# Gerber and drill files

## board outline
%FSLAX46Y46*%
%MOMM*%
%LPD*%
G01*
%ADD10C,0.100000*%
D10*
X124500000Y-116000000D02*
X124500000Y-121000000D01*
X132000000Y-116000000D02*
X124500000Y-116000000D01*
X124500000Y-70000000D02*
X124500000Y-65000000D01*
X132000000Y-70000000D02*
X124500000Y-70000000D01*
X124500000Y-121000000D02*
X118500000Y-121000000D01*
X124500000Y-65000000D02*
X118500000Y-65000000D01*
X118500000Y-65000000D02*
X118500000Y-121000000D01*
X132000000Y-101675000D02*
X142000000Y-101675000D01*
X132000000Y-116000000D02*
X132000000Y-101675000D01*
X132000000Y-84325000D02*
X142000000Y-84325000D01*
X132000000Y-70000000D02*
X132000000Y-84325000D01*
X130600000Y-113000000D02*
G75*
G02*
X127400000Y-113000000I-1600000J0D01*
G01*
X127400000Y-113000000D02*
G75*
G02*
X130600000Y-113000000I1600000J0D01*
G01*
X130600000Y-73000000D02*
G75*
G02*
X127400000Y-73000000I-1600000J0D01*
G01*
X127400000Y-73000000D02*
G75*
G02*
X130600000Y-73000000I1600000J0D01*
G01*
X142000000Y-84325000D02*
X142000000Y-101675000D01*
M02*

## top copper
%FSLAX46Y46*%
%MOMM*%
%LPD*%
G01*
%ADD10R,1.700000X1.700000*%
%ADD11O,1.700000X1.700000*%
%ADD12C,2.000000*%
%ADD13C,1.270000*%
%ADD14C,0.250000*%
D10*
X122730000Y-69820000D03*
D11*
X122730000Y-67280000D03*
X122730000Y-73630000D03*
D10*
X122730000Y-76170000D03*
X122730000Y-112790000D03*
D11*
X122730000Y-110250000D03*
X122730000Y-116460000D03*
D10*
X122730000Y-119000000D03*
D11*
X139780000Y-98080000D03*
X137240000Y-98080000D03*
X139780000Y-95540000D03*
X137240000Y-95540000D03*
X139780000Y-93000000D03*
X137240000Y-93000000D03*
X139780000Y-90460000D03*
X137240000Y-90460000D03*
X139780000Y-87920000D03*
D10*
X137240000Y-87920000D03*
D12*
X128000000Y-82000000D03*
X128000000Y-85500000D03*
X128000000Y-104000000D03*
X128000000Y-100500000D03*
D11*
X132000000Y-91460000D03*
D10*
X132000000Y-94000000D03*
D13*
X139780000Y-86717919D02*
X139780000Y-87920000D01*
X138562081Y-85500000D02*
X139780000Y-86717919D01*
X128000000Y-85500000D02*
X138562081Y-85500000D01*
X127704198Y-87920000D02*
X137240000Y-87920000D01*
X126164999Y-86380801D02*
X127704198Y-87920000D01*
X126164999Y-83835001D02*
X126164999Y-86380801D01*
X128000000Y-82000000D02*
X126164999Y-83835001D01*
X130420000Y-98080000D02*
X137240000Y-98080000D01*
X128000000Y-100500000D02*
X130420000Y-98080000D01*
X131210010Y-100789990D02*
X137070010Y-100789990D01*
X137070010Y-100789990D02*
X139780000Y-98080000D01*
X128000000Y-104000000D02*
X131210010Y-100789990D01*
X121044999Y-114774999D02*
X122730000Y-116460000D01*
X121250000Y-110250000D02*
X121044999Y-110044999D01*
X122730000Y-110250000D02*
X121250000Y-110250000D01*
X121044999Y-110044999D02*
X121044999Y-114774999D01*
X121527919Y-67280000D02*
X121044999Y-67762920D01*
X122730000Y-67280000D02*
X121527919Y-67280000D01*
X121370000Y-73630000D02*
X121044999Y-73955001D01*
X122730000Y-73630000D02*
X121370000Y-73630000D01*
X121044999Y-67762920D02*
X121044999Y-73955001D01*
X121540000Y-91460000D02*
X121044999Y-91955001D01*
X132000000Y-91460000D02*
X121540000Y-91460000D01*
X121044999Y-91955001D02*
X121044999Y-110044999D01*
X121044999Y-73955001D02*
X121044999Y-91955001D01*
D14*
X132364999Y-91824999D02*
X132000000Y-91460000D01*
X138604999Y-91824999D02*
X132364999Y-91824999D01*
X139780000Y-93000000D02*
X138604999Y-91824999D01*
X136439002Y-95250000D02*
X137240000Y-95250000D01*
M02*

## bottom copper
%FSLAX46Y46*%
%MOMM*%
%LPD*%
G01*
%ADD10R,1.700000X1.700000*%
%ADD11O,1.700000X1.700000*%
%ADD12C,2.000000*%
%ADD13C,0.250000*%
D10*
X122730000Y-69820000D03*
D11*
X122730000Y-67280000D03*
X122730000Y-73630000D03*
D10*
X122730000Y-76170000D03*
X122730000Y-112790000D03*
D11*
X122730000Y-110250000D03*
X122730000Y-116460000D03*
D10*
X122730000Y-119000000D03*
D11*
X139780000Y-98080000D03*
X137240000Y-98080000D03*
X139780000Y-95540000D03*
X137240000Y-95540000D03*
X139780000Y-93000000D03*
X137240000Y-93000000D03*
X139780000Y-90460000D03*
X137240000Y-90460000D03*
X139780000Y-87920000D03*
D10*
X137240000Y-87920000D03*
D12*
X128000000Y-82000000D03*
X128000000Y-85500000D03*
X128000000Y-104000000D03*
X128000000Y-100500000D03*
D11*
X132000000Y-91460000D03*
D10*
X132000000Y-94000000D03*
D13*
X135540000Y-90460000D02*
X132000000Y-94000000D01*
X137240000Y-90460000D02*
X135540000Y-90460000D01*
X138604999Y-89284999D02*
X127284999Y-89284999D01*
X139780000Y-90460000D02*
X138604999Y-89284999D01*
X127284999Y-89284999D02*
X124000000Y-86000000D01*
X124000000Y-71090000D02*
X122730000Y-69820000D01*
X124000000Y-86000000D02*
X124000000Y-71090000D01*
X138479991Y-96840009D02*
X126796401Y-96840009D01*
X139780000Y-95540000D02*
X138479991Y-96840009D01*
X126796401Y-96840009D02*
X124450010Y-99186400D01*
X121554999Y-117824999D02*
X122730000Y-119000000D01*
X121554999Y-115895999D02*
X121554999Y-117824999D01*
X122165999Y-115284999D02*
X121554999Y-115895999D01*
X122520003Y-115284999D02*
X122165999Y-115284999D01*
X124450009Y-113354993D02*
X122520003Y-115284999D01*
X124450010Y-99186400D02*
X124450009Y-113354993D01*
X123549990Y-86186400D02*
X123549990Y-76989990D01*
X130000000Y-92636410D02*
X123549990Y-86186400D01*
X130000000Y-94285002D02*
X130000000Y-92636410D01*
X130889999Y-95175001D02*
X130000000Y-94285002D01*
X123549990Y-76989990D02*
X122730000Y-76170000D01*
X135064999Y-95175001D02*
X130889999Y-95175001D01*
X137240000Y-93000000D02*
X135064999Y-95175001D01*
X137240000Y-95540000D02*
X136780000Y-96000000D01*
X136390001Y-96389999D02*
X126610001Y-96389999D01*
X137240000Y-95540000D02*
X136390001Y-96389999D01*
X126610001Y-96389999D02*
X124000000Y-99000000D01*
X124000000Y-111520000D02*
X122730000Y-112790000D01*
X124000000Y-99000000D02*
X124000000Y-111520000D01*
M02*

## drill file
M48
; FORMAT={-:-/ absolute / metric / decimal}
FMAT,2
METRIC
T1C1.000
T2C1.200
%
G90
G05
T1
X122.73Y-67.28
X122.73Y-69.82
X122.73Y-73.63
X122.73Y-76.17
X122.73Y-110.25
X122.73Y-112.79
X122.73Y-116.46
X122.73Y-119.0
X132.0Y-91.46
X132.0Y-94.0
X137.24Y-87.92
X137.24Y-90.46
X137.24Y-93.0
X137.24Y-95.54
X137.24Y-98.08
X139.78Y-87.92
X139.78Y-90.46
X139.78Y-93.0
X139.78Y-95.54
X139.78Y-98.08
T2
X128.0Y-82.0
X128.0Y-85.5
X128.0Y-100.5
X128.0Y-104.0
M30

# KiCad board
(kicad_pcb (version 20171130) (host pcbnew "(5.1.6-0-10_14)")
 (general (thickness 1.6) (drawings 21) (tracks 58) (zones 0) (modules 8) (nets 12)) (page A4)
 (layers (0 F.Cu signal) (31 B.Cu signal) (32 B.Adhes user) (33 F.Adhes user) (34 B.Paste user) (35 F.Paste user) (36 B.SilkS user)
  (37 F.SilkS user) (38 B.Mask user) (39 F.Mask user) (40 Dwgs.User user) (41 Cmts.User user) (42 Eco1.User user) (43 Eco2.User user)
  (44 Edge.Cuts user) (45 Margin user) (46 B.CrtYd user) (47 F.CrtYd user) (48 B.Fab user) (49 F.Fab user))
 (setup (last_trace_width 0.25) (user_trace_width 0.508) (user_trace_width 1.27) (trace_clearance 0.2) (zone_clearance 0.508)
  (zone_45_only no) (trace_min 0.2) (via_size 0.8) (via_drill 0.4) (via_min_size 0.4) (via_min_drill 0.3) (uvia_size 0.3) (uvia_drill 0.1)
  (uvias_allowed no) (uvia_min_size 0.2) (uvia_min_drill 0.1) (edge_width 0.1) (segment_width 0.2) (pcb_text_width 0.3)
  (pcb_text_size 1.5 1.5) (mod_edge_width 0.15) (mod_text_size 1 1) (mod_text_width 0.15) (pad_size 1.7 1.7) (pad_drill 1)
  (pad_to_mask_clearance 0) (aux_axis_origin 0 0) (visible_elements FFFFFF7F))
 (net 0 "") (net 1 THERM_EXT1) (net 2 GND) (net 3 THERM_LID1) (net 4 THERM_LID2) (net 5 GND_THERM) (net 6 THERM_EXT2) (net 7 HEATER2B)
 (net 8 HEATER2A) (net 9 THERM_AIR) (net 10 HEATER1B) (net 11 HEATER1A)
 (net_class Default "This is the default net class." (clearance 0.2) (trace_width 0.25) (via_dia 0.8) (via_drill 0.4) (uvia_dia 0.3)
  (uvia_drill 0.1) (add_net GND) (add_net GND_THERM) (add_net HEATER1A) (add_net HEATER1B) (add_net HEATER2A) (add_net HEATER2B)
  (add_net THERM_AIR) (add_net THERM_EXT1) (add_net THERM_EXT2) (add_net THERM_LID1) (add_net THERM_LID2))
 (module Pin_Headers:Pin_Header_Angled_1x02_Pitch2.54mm (layer F.Cu) (at 122.73 69.82 180)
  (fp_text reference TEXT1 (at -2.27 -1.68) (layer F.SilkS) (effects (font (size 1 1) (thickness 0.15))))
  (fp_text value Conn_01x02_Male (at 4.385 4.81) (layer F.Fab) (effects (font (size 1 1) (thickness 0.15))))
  (pad 1 thru_hole rect (at 0 0 180) (size 1.7 1.7) (drill 1) (layers *.Cu *.Mask) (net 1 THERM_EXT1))
  (pad 2 thru_hole oval (at 0 2.54 180) (size 1.7 1.7) (drill 1) (layers *.Cu *.Mask) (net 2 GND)))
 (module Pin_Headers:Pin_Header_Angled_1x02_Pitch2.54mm (layer F.Cu) (at 122.73 76.17 180)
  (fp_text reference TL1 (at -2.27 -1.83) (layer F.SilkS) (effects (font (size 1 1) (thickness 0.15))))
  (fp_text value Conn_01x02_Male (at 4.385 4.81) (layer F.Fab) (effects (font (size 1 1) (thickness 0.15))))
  (pad 2 thru_hole oval (at 0 2.54 180) (size 1.7 1.7) (drill 1) (layers *.Cu *.Mask) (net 2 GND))
  (pad 1 thru_hole rect (at 0 0 180) (size 1.7 1.7) (drill 1) (layers *.Cu *.Mask) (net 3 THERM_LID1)))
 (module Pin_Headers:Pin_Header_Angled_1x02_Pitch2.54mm (layer F.Cu) (at 122.73 112.79 180)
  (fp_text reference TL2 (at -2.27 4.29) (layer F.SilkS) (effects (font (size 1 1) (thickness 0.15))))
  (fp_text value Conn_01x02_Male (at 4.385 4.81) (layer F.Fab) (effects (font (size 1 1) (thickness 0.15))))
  (pad 1 thru_hole rect (at 0 0 180) (size 1.7 1.7) (drill 1) (layers *.Cu *.Mask) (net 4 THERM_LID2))
  (pad 2 thru_hole oval (at 0 2.54 180) (size 1.7 1.7) (drill 1) (layers *.Cu *.Mask) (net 2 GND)))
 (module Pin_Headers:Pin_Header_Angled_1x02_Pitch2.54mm (layer F.Cu) (at 122.73 119 180)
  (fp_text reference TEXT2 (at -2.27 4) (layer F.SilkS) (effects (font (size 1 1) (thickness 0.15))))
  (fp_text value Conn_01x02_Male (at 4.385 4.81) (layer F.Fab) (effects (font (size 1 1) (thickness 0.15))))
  (pad 2 thru_hole oval (at 0 2.54 180) (size 1.7 1.7) (drill 1) (layers *.Cu *.Mask) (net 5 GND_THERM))
  (pad 1 thru_hole rect (at 0 0 180) (size 1.7 1.7) (drill 1) (layers *.Cu *.Mask) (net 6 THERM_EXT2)))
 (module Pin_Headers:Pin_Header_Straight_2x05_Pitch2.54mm (layer F.Cu) (at 137.24 87.92)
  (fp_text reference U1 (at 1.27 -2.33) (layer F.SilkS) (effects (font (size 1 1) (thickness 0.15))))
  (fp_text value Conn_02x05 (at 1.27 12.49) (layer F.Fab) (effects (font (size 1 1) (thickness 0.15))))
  (pad 10 thru_hole oval (at 2.54 10.16) (size 1.7 1.7) (drill 1) (layers *.Cu *.Mask) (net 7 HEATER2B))
  (pad 9 thru_hole oval (at 0 10.16) (size 1.7 1.7) (drill 1) (layers *.Cu *.Mask) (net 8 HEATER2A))
  (pad 8 thru_hole oval (at 2.54 7.62) (size 1.7 1.7) (drill 1) (layers *.Cu *.Mask) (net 6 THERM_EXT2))
  (pad 7 thru_hole oval (at 0 7.62) (size 1.7 1.7) (drill 1) (layers *.Cu *.Mask) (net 4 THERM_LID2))
  (pad 6 thru_hole oval (at 2.54 5.08) (size 1.7 1.7) (drill 1) (layers *.Cu *.Mask) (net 2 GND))
  (pad 5 thru_hole oval (at 0 5.08) (size 1.7 1.7) (drill 1) (layers *.Cu *.Mask) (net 3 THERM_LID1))
  (pad 4 thru_hole oval (at 2.54 2.54) (size 1.7 1.7) (drill 1) (layers *.Cu *.Mask) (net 1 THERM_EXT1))
  (pad 3 thru_hole oval (at 0 2.54) (size 1.7 1.7) (drill 1) (layers *.Cu *.Mask) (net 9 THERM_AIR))
  (pad 2 thru_hole oval (at 2.54 0) (size 1.7 1.7) (drill 1) (layers *.Cu *.Mask) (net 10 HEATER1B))
  (pad 1 thru_hole rect (at 0 0) (size 1.7 1.7) (drill 1) (layers *.Cu *.Mask) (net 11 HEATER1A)))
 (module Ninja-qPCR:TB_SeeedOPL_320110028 (layer F.Cu) (at 128 82 270)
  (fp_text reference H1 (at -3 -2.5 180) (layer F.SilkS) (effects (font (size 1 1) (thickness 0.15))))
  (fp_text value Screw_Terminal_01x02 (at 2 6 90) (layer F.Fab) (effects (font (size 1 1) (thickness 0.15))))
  (pad 1 thru_hole circle (at 0 0 270) (size 2 2) (drill 1.2) (layers *.Cu *.Mask) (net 11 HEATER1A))
  (pad 2 thru_hole circle (at 3.5 0 270) (size 2 2) (drill 1.2) (layers *.Cu *.Mask) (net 10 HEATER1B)))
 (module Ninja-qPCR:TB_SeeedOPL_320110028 (layer F.Cu) (at 128 100.5 270)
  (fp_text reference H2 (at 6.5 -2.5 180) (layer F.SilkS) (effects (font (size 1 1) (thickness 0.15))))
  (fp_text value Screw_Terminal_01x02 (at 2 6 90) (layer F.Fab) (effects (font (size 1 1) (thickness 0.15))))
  (pad 2 thru_hole circle (at 3.5 0 270) (size 2 2) (drill 1.2) (layers *.Cu *.Mask) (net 7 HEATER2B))
  (pad 1 thru_hole circle (at 0 0 270) (size 2 2) (drill 1.2) (layers *.Cu *.Mask) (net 8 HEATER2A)))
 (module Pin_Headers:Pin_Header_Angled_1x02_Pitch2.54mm (layer F.Cu) (at 132 94 180)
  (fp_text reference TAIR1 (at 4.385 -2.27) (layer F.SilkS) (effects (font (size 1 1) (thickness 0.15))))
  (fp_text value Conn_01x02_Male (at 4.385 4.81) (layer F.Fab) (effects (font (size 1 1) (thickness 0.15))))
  (pad 2 thru_hole oval (at 0 2.54 180) (size 1.7 1.7) (drill 1) (layers *.Cu *.Mask) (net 2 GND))
  (pad 1 thru_hole rect (at 0 0 180) (size 1.7 1.7) (drill 1) (layers *.Cu *.Mask) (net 9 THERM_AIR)))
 (gr_line (start 124.5 116) (end 124.5 121) (layer Edge.Cuts) (width 0.1))
 (gr_line (start 132 116) (end 124.5 116) (layer Edge.Cuts) (width 0.1))
 (gr_line (start 124.5 70) (end 124.5 65) (layer Edge.Cuts) (width 0.1))
 (gr_line (start 132 70) (end 124.5 70) (layer Edge.Cuts) (width 0.1))
 (gr_line (start 124.5 121) (end 118.5 121) (layer Edge.Cuts) (width 0.1))
 (gr_line (start 124.5 65) (end 118.5 65) (layer Edge.Cuts) (width 0.1))
 (gr_line (start 118.5 65) (end 118.5 121) (layer Edge.Cuts) (width 0.1))
 (gr_line (start 132 101.675) (end 142 101.675) (layer Edge.Cuts) (width 0.1))
 (gr_line (start 132 116) (end 132 101.675) (layer Edge.Cuts) (width 0.1))
 (gr_line (start 132 84.325) (end 142 84.325) (layer Edge.Cuts) (width 0.1))
 (gr_line (start 132 70) (end 132 84.325) (layer Edge.Cuts) (width 0.1))
 (gr_circle (center 129 113) (end 130.6 113) (layer Edge.Cuts) (width 0.1))
 (gr_circle (center 129 73) (end 130.6 73) (layer Edge.Cuts) (width 0.1))
 (gr_line (start 142 84.325) (end 142 101.675) (layer Edge.Cuts) (width 0.1))
 (segment (start 139.78 86.717919) (end 139.78 87.92) (width 1.27) (layer F.Cu) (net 10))
 (segment (start 138.562081 85.5) (end 139.78 86.717919) (width 1.27) (layer F.Cu) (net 10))
 (segment (start 128 85.5) (end 138.562081 85.5) (width 1.27) (layer F.Cu) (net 10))
 (segment (start 127.704198 87.92) (end 137.24 87.92) (width 1.27) (layer F.Cu) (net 11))
 (segment (start 126.164999 86.380801) (end 127.704198 87.92) (width 1.27) (layer F.Cu) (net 11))
 (segment (start 126.164999 83.835001) (end 126.164999 86.380801) (width 1.27) (layer F.Cu) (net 11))
 (segment (start 128 82) (end 126.164999 83.835001) (width 1.27) (layer F.Cu) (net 11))
 (segment (start 130.42 98.08) (end 137.24 98.08) (width 1.27) (layer F.Cu) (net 8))
 (segment (start 128 100.5) (end 130.42 98.08) (width 1.27) (layer F.Cu) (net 8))
 (segment (start 131.21001 100.78999) (end 137.07001 100.78999) (width 1.27) (layer F.Cu) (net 7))
 (segment (start 137.07001 100.78999) (end 139.78 98.08) (width 1.27) (layer F.Cu) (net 7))
 (segment (start 128 104) (end 131.21001 100.78999) (width 1.27) (layer F.Cu) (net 7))
 (segment (start 135.54 90.46) (end 132 94) (width 0.25) (layer B.Cu) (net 9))
 (segment (start 137.24 90.46) (end 135.54 90.46) (width 0.25) (layer B.Cu) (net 9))
 (segment (start 121.044999 114.774999) (end 122.73 116.46) (width 1.27) (layer F.Cu) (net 5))
 (segment (start 121.25 110.25) (end 121.044999 110.044999) (width 1.27) (layer F.Cu) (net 5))
 (segment (start 122.73 110.25) (end 121.25 110.25) (width 1.27) (layer F.Cu) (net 5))
 (segment (start 121.044999 110.044999) (end 121.044999 114.774999) (width 1.27) (layer F.Cu) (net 5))
 (segment (start 121.527919 67.28) (end 121.044999 67.76292) (width 1.27) (layer F.Cu) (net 5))
 (segment (start 122.73 67.28) (end 121.527919 67.28) (width 1.27) (layer F.Cu) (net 5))
 (segment (start 121.37 73.63) (end 121.044999 73.955001) (width 1.27) (layer F.Cu) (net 5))
 (segment (start 122.73 73.63) (end 121.37 73.63) (width 1.27) (layer F.Cu) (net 5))
 (segment (start 121.044999 67.76292) (end 121.044999 73.955001) (width 1.27) (layer F.Cu) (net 5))
 (segment (start 121.54 91.46) (end 121.044999 91.955001) (width 1.27) (layer F.Cu) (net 5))
 (segment (start 132 91.46) (end 121.54 91.46) (width 1.27) (layer F.Cu) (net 5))
 (segment (start 121.044999 91.955001) (end 121.044999 110.044999) (width 1.27) (layer F.Cu) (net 5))
 (segment (start 121.044999 73.955001) (end 121.044999 91.955001) (width 1.27) (layer F.Cu) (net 5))
 (segment (start 132.364999 91.824999) (end 132 91.46) (width 0.25) (layer F.Cu) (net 5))
 (segment (start 138.604999 91.824999) (end 132.364999 91.824999) (width 0.25) (layer F.Cu) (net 5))
 (segment (start 139.78 93) (end 138.604999 91.824999) (width 0.25) (layer F.Cu) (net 5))
 (segment (start 138.604999 89.284999) (end 127.284999 89.284999) (width 0.25) (layer B.Cu) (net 1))
 (segment (start 139.78 90.46) (end 138.604999 89.284999) (width 0.25) (layer B.Cu) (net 1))
 (segment (start 127.284999 89.284999) (end 124 86) (width 0.25) (layer B.Cu) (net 1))
 (segment (start 124 71.09) (end 122.73 69.82) (width 0.25) (layer B.Cu) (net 1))
 (segment (start 124 86) (end 124 71.09) (width 0.25) (layer B.Cu) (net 1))
 (segment (start 138.479991 96.840009) (end 126.796401 96.840009) (width 0.25) (layer B.Cu) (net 6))
 (segment (start 139.78 95.54) (end 138.479991 96.840009) (width 0.25) (layer B.Cu) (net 6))
 (segment (start 126.796401 96.840009) (end 124.45001 99.1864) (width 0.25) (layer B.Cu) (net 6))
 (segment (start 121.554999 117.824999) (end 122.73 119) (width 0.25) (layer B.Cu) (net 6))
 (segment (start 121.554999 115.895999) (end 121.554999 117.824999) (width 0.25) (layer B.Cu) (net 6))
 (segment (start 122.165999 115.284999) (end 121.554999 115.895999) (width 0.25) (layer B.Cu) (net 6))
 (segment (start 122.520003 115.284999) (end 122.165999 115.284999) (width 0.25) (layer B.Cu) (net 6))
 (segment (start 124.450009 113.354993) (end 122.520003 115.284999) (width 0.25) (layer B.Cu) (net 6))
 (segment (start 124.45001 99.1864) (end 124.450009 113.354993) (width 0.25) (layer B.Cu) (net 6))
 (segment (start 123.54999 86.1864) (end 123.54999 76.98999) (width 0.25) (layer B.Cu) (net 3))
 (segment (start 130 92.63641) (end 123.54999 86.1864) (width 0.25) (layer B.Cu) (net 3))
 (segment (start 130 94.285002) (end 130 92.63641) (width 0.25) (layer B.Cu) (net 3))
 (segment (start 130.889999 95.175001) (end 130 94.285002) (width 0.25) (layer B.Cu) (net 3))
 (segment (start 123.54999 76.98999) (end 122.73 76.17) (width 0.25) (layer B.Cu) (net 3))
 (segment (start 135.064999 95.175001) (end 130.889999 95.175001) (width 0.25) (layer B.Cu) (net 3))
 (segment (start 137.24 93) (end 135.064999 95.175001) (width 0.25) (layer B.Cu) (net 3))
 (segment (start 136.439002 95.25) (end 137.24 95.25) (width 0.25) (layer F.Cu) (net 4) (status 20))
 (segment (start 137.24 95.54) (end 136.78 96) (width 0.25) (layer B.Cu) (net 4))
 (segment (start 136.390001 96.389999) (end 126.610001 96.389999) (width 0.25) (layer B.Cu) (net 4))
 (segment (start 137.24 95.54) (end 136.390001 96.389999) (width 0.25) (layer B.Cu) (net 4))
 (segment (start 126.610001 96.389999) (end 124 99) (width 0.25) (layer B.Cu) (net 4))
 (segment (start 124 111.52) (end 122.73 112.79) (width 0.25) (layer B.Cu) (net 4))
 (segment (start 124 99) (end 124 111.52) (width 0.25) (layer B.Cu) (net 4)))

